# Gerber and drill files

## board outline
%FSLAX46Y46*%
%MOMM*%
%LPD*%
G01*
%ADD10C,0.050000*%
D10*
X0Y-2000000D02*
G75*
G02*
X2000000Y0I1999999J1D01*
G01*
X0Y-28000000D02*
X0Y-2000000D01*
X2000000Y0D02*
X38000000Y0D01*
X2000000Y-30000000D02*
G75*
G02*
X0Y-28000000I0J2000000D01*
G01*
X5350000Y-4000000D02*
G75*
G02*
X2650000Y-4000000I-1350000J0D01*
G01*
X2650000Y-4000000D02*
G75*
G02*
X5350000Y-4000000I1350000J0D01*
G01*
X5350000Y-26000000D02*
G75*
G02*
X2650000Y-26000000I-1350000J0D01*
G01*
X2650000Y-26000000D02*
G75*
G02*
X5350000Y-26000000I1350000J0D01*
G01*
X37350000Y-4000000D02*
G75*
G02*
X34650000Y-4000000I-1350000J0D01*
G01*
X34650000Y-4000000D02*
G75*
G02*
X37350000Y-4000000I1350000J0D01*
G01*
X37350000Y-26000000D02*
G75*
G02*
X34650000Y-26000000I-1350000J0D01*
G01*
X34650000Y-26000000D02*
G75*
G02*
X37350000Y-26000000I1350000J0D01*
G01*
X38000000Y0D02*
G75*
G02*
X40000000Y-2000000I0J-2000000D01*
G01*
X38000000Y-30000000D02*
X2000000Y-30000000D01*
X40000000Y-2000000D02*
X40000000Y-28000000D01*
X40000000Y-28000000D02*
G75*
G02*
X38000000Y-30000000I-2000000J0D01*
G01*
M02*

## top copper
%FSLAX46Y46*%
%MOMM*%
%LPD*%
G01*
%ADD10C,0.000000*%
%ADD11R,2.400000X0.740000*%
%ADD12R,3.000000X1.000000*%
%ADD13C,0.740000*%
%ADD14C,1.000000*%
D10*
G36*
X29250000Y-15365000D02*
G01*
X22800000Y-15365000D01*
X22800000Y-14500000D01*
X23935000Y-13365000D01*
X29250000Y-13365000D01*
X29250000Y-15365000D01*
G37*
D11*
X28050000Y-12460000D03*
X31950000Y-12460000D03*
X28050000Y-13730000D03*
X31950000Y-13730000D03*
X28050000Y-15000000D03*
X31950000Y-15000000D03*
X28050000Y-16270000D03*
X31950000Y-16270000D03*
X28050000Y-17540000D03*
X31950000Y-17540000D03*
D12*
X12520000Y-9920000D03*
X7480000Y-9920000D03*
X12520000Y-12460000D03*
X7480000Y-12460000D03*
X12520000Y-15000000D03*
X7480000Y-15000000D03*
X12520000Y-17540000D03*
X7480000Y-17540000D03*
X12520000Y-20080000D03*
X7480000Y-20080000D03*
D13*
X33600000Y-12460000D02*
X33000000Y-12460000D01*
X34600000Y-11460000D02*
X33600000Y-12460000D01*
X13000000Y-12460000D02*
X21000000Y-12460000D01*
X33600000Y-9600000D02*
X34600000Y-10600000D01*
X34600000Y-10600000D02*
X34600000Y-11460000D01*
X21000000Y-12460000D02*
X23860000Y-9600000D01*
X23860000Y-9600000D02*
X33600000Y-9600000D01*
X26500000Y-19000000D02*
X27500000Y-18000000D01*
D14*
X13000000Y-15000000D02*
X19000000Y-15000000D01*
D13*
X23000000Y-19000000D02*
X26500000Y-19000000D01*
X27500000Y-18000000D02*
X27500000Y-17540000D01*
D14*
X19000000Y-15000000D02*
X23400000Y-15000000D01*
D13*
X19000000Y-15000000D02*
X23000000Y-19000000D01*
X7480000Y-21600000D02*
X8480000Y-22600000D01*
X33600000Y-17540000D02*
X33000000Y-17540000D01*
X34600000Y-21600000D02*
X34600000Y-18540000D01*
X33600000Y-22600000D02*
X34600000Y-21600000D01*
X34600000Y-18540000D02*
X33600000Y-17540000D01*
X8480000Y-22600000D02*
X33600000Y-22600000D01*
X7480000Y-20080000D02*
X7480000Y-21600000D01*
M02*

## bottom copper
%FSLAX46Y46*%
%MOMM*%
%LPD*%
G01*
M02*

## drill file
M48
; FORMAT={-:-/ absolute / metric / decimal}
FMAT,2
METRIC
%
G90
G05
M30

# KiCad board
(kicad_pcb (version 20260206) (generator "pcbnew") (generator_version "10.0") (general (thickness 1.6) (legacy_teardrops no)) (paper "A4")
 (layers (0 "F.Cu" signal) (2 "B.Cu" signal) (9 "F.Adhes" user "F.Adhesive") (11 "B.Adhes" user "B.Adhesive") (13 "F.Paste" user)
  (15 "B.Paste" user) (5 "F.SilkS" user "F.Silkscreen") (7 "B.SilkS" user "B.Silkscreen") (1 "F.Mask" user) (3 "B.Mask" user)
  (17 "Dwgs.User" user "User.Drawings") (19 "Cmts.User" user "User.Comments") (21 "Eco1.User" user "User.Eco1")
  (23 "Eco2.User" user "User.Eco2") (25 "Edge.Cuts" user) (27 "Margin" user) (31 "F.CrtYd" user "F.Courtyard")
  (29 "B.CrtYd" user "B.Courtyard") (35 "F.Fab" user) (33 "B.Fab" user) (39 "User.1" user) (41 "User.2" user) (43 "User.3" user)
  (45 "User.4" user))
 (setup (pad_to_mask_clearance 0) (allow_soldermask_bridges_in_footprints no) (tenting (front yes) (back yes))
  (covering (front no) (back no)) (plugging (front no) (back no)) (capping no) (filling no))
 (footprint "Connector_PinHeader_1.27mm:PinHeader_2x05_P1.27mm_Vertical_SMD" (layer "F.Cu") (at 30 15)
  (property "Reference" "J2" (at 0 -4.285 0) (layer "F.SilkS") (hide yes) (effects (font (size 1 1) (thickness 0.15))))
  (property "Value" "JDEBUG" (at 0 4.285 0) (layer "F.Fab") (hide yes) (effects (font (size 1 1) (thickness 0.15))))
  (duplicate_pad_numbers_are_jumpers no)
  (pad "1" smd rect (at -1.95 -2.54) (size 2.4 0.74) (layers "F.Cu" "F.Mask" "F.Paste"))
  (pad "2" smd rect (at 1.95 -2.54) (size 2.4 0.74) (layers "F.Cu" "F.Mask" "F.Paste") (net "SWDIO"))
  (pad "3" smd rect (at -1.95 -1.27) (size 2.4 0.74) (layers "F.Cu" "F.Mask" "F.Paste") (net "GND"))
  (pad "4" smd rect (at 1.95 -1.27) (size 2.4 0.74) (layers "F.Cu" "F.Mask" "F.Paste"))
  (pad "5" smd rect (at -1.95 0) (size 2.4 0.74) (layers "F.Cu" "F.Mask" "F.Paste") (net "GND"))
  (pad "6" smd rect (at 1.95 0) (size 2.4 0.74) (layers "F.Cu" "F.Mask" "F.Paste"))
  (pad "7" smd rect (at -1.95 1.27) (size 2.4 0.74) (layers "F.Cu" "F.Mask" "F.Paste"))
  (pad "8" smd rect (at 1.95 1.27) (size 2.4 0.74) (layers "F.Cu" "F.Mask" "F.Paste"))
  (pad "9" smd rect (at -1.95 2.54) (size 2.4 0.74) (layers "F.Cu" "F.Mask" "F.Paste") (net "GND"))
  (pad "10" smd rect (at 1.95 2.54) (size 2.4 0.74) (layers "F.Cu" "F.Mask" "F.Paste") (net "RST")))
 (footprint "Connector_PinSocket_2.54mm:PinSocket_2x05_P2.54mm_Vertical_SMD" (layer "F.Cu") (at 10 15)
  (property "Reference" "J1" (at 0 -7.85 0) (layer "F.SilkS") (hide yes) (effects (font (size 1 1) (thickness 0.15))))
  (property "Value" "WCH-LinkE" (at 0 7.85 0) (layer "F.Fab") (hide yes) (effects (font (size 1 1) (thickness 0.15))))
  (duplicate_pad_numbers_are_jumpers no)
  (pad "1" smd rect (at 2.52 -5.08) (size 3 1) (layers "F.Cu" "F.Mask" "F.Paste"))
  (pad "2" smd rect (at -2.52 -5.08) (size 3 1) (layers "F.Cu" "F.Mask" "F.Paste"))
  (pad "3" smd rect (at 2.52 -2.54) (size 3 1) (layers "F.Cu" "F.Mask" "F.Paste") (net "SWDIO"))
  (pad "4" smd rect (at -2.52 -2.54) (size 3 1) (layers "F.Cu" "F.Mask" "F.Paste"))
  (pad "5" smd rect (at 2.52 0) (size 3 1) (layers "F.Cu" "F.Mask" "F.Paste") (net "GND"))
  (pad "6" smd rect (at -2.52 0) (size 3 1) (layers "F.Cu" "F.Mask" "F.Paste"))
  (pad "7" smd rect (at 2.52 2.54) (size 3 1) (layers "F.Cu" "F.Mask" "F.Paste"))
  (pad "8" smd rect (at -2.52 2.54) (size 3 1) (layers "F.Cu" "F.Mask" "F.Paste"))
  (pad "9" smd rect (at 2.52 5.08) (size 3 1) (layers "F.Cu" "F.Mask" "F.Paste"))
  (pad "10" smd rect (at -2.52 5.08) (size 3 1) (layers "F.Cu" "F.Mask" "F.Paste") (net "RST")))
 (gr_poly
  (pts (xy 22.8 14.5) (xy 23.935 13.365) (xy 29.25 13.365) (xy 29.25 15.365) (xy 22.8 15.365)) (stroke (width 0) (type default)) (fill yes)
  (layer "F.Cu") (net "GND"))
 (gr_arc (start 0 2) (mid 0.585786 0.585786) (end 2 0) (stroke (width 0.05) (type default)) (layer "Edge.Cuts"))
 (gr_line (start 0 28) (end 0 2) (stroke (width 0.05) (type default)) (layer "Edge.Cuts"))
 (gr_line (start 2 0) (end 38 0) (stroke (width 0.05) (type default)) (layer "Edge.Cuts"))
 (gr_arc (start 2 30) (mid 0.585786 29.414213) (end 0 28) (stroke (width 0.05) (type default)) (layer "Edge.Cuts"))
 (gr_circle (center 4 4) (end 5.35 4) (stroke (width 0.05) (type default)) (fill no) (layer "Edge.Cuts"))
 (gr_circle (center 4 26) (end 5.35 26) (stroke (width 0.05) (type default)) (fill no) (layer "Edge.Cuts"))
 (gr_circle (center 36 4) (end 37.35 4) (stroke (width 0.05) (type default)) (fill no) (layer "Edge.Cuts"))
 (gr_circle (center 36 26) (end 37.35 26) (stroke (width 0.05) (type default)) (fill no) (layer "Edge.Cuts"))
 (gr_arc (start 38 0) (mid 39.414213 0.585786) (end 40 2) (stroke (width 0.05) (type default)) (layer "Edge.Cuts"))
 (gr_line (start 38 30) (end 2 30) (stroke (width 0.05) (type default)) (layer "Edge.Cuts"))
 (gr_line (start 40 2) (end 40 28) (stroke (width 0.05) (type default)) (layer "Edge.Cuts"))
 (gr_arc (start 40 28) (mid 39.414213 29.414213) (end 38 30) (stroke (width 0.05) (type default)) (layer "Edge.Cuts"))
 (segment (start 33.6 12.46) (end 33 12.46) (width 0.74) (layer "F.Cu") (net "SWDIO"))
 (segment (start 34.6 11.46) (end 33.6 12.46) (width 0.74) (layer "F.Cu") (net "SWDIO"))
 (segment (start 13 12.46) (end 21 12.46) (width 0.74) (layer "F.Cu") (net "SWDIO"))
 (segment (start 33.6 9.6) (end 34.6 10.6) (width 0.74) (layer "F.Cu") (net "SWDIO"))
 (segment (start 34.6 10.6) (end 34.6 11.46) (width 0.74) (layer "F.Cu") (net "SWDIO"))
 (segment (start 21 12.46) (end 23.86 9.6) (width 0.74) (layer "F.Cu") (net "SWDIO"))
 (segment (start 23.86 9.6) (end 33.6 9.6) (width 0.74) (layer "F.Cu") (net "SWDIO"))
 (segment (start 26.5 19) (end 27.5 18) (width 0.74) (layer "F.Cu") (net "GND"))
 (segment (start 13 15) (end 19 15) (width 1) (layer "F.Cu") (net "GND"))
 (segment (start 23 19) (end 26.5 19) (width 0.74) (layer "F.Cu") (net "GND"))
 (segment (start 27.5 18) (end 27.5 17.54) (width 0.74) (layer "F.Cu") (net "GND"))
 (segment (start 19 15) (end 23.4 15) (width 1) (layer "F.Cu") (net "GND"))
 (segment (start 19 15) (end 23 19) (width 0.74) (layer "F.Cu") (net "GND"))
 (segment (start 7.48 21.6) (end 8.48 22.6) (width 0.74) (layer "F.Cu") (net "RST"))
 (segment (start 33.6 17.54) (end 33 17.54) (width 0.74) (layer "F.Cu") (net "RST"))
 (segment (start 34.6 21.6) (end 34.6 18.54) (width 0.74) (layer "F.Cu") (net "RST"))
 (segment (start 33.6 22.6) (end 34.6 21.6) (width 0.74) (layer "F.Cu") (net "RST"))
 (segment (start 34.6 18.54) (end 33.6 17.54) (width 0.74) (layer "F.Cu") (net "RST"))
 (segment (start 8.48 22.6) (end 33.6 22.6) (width 0.74) (layer "F.Cu") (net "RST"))
 (segment (start 7.48 20.08) (end 7.48 21.6) (width 0.74) (layer "F.Cu") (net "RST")))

